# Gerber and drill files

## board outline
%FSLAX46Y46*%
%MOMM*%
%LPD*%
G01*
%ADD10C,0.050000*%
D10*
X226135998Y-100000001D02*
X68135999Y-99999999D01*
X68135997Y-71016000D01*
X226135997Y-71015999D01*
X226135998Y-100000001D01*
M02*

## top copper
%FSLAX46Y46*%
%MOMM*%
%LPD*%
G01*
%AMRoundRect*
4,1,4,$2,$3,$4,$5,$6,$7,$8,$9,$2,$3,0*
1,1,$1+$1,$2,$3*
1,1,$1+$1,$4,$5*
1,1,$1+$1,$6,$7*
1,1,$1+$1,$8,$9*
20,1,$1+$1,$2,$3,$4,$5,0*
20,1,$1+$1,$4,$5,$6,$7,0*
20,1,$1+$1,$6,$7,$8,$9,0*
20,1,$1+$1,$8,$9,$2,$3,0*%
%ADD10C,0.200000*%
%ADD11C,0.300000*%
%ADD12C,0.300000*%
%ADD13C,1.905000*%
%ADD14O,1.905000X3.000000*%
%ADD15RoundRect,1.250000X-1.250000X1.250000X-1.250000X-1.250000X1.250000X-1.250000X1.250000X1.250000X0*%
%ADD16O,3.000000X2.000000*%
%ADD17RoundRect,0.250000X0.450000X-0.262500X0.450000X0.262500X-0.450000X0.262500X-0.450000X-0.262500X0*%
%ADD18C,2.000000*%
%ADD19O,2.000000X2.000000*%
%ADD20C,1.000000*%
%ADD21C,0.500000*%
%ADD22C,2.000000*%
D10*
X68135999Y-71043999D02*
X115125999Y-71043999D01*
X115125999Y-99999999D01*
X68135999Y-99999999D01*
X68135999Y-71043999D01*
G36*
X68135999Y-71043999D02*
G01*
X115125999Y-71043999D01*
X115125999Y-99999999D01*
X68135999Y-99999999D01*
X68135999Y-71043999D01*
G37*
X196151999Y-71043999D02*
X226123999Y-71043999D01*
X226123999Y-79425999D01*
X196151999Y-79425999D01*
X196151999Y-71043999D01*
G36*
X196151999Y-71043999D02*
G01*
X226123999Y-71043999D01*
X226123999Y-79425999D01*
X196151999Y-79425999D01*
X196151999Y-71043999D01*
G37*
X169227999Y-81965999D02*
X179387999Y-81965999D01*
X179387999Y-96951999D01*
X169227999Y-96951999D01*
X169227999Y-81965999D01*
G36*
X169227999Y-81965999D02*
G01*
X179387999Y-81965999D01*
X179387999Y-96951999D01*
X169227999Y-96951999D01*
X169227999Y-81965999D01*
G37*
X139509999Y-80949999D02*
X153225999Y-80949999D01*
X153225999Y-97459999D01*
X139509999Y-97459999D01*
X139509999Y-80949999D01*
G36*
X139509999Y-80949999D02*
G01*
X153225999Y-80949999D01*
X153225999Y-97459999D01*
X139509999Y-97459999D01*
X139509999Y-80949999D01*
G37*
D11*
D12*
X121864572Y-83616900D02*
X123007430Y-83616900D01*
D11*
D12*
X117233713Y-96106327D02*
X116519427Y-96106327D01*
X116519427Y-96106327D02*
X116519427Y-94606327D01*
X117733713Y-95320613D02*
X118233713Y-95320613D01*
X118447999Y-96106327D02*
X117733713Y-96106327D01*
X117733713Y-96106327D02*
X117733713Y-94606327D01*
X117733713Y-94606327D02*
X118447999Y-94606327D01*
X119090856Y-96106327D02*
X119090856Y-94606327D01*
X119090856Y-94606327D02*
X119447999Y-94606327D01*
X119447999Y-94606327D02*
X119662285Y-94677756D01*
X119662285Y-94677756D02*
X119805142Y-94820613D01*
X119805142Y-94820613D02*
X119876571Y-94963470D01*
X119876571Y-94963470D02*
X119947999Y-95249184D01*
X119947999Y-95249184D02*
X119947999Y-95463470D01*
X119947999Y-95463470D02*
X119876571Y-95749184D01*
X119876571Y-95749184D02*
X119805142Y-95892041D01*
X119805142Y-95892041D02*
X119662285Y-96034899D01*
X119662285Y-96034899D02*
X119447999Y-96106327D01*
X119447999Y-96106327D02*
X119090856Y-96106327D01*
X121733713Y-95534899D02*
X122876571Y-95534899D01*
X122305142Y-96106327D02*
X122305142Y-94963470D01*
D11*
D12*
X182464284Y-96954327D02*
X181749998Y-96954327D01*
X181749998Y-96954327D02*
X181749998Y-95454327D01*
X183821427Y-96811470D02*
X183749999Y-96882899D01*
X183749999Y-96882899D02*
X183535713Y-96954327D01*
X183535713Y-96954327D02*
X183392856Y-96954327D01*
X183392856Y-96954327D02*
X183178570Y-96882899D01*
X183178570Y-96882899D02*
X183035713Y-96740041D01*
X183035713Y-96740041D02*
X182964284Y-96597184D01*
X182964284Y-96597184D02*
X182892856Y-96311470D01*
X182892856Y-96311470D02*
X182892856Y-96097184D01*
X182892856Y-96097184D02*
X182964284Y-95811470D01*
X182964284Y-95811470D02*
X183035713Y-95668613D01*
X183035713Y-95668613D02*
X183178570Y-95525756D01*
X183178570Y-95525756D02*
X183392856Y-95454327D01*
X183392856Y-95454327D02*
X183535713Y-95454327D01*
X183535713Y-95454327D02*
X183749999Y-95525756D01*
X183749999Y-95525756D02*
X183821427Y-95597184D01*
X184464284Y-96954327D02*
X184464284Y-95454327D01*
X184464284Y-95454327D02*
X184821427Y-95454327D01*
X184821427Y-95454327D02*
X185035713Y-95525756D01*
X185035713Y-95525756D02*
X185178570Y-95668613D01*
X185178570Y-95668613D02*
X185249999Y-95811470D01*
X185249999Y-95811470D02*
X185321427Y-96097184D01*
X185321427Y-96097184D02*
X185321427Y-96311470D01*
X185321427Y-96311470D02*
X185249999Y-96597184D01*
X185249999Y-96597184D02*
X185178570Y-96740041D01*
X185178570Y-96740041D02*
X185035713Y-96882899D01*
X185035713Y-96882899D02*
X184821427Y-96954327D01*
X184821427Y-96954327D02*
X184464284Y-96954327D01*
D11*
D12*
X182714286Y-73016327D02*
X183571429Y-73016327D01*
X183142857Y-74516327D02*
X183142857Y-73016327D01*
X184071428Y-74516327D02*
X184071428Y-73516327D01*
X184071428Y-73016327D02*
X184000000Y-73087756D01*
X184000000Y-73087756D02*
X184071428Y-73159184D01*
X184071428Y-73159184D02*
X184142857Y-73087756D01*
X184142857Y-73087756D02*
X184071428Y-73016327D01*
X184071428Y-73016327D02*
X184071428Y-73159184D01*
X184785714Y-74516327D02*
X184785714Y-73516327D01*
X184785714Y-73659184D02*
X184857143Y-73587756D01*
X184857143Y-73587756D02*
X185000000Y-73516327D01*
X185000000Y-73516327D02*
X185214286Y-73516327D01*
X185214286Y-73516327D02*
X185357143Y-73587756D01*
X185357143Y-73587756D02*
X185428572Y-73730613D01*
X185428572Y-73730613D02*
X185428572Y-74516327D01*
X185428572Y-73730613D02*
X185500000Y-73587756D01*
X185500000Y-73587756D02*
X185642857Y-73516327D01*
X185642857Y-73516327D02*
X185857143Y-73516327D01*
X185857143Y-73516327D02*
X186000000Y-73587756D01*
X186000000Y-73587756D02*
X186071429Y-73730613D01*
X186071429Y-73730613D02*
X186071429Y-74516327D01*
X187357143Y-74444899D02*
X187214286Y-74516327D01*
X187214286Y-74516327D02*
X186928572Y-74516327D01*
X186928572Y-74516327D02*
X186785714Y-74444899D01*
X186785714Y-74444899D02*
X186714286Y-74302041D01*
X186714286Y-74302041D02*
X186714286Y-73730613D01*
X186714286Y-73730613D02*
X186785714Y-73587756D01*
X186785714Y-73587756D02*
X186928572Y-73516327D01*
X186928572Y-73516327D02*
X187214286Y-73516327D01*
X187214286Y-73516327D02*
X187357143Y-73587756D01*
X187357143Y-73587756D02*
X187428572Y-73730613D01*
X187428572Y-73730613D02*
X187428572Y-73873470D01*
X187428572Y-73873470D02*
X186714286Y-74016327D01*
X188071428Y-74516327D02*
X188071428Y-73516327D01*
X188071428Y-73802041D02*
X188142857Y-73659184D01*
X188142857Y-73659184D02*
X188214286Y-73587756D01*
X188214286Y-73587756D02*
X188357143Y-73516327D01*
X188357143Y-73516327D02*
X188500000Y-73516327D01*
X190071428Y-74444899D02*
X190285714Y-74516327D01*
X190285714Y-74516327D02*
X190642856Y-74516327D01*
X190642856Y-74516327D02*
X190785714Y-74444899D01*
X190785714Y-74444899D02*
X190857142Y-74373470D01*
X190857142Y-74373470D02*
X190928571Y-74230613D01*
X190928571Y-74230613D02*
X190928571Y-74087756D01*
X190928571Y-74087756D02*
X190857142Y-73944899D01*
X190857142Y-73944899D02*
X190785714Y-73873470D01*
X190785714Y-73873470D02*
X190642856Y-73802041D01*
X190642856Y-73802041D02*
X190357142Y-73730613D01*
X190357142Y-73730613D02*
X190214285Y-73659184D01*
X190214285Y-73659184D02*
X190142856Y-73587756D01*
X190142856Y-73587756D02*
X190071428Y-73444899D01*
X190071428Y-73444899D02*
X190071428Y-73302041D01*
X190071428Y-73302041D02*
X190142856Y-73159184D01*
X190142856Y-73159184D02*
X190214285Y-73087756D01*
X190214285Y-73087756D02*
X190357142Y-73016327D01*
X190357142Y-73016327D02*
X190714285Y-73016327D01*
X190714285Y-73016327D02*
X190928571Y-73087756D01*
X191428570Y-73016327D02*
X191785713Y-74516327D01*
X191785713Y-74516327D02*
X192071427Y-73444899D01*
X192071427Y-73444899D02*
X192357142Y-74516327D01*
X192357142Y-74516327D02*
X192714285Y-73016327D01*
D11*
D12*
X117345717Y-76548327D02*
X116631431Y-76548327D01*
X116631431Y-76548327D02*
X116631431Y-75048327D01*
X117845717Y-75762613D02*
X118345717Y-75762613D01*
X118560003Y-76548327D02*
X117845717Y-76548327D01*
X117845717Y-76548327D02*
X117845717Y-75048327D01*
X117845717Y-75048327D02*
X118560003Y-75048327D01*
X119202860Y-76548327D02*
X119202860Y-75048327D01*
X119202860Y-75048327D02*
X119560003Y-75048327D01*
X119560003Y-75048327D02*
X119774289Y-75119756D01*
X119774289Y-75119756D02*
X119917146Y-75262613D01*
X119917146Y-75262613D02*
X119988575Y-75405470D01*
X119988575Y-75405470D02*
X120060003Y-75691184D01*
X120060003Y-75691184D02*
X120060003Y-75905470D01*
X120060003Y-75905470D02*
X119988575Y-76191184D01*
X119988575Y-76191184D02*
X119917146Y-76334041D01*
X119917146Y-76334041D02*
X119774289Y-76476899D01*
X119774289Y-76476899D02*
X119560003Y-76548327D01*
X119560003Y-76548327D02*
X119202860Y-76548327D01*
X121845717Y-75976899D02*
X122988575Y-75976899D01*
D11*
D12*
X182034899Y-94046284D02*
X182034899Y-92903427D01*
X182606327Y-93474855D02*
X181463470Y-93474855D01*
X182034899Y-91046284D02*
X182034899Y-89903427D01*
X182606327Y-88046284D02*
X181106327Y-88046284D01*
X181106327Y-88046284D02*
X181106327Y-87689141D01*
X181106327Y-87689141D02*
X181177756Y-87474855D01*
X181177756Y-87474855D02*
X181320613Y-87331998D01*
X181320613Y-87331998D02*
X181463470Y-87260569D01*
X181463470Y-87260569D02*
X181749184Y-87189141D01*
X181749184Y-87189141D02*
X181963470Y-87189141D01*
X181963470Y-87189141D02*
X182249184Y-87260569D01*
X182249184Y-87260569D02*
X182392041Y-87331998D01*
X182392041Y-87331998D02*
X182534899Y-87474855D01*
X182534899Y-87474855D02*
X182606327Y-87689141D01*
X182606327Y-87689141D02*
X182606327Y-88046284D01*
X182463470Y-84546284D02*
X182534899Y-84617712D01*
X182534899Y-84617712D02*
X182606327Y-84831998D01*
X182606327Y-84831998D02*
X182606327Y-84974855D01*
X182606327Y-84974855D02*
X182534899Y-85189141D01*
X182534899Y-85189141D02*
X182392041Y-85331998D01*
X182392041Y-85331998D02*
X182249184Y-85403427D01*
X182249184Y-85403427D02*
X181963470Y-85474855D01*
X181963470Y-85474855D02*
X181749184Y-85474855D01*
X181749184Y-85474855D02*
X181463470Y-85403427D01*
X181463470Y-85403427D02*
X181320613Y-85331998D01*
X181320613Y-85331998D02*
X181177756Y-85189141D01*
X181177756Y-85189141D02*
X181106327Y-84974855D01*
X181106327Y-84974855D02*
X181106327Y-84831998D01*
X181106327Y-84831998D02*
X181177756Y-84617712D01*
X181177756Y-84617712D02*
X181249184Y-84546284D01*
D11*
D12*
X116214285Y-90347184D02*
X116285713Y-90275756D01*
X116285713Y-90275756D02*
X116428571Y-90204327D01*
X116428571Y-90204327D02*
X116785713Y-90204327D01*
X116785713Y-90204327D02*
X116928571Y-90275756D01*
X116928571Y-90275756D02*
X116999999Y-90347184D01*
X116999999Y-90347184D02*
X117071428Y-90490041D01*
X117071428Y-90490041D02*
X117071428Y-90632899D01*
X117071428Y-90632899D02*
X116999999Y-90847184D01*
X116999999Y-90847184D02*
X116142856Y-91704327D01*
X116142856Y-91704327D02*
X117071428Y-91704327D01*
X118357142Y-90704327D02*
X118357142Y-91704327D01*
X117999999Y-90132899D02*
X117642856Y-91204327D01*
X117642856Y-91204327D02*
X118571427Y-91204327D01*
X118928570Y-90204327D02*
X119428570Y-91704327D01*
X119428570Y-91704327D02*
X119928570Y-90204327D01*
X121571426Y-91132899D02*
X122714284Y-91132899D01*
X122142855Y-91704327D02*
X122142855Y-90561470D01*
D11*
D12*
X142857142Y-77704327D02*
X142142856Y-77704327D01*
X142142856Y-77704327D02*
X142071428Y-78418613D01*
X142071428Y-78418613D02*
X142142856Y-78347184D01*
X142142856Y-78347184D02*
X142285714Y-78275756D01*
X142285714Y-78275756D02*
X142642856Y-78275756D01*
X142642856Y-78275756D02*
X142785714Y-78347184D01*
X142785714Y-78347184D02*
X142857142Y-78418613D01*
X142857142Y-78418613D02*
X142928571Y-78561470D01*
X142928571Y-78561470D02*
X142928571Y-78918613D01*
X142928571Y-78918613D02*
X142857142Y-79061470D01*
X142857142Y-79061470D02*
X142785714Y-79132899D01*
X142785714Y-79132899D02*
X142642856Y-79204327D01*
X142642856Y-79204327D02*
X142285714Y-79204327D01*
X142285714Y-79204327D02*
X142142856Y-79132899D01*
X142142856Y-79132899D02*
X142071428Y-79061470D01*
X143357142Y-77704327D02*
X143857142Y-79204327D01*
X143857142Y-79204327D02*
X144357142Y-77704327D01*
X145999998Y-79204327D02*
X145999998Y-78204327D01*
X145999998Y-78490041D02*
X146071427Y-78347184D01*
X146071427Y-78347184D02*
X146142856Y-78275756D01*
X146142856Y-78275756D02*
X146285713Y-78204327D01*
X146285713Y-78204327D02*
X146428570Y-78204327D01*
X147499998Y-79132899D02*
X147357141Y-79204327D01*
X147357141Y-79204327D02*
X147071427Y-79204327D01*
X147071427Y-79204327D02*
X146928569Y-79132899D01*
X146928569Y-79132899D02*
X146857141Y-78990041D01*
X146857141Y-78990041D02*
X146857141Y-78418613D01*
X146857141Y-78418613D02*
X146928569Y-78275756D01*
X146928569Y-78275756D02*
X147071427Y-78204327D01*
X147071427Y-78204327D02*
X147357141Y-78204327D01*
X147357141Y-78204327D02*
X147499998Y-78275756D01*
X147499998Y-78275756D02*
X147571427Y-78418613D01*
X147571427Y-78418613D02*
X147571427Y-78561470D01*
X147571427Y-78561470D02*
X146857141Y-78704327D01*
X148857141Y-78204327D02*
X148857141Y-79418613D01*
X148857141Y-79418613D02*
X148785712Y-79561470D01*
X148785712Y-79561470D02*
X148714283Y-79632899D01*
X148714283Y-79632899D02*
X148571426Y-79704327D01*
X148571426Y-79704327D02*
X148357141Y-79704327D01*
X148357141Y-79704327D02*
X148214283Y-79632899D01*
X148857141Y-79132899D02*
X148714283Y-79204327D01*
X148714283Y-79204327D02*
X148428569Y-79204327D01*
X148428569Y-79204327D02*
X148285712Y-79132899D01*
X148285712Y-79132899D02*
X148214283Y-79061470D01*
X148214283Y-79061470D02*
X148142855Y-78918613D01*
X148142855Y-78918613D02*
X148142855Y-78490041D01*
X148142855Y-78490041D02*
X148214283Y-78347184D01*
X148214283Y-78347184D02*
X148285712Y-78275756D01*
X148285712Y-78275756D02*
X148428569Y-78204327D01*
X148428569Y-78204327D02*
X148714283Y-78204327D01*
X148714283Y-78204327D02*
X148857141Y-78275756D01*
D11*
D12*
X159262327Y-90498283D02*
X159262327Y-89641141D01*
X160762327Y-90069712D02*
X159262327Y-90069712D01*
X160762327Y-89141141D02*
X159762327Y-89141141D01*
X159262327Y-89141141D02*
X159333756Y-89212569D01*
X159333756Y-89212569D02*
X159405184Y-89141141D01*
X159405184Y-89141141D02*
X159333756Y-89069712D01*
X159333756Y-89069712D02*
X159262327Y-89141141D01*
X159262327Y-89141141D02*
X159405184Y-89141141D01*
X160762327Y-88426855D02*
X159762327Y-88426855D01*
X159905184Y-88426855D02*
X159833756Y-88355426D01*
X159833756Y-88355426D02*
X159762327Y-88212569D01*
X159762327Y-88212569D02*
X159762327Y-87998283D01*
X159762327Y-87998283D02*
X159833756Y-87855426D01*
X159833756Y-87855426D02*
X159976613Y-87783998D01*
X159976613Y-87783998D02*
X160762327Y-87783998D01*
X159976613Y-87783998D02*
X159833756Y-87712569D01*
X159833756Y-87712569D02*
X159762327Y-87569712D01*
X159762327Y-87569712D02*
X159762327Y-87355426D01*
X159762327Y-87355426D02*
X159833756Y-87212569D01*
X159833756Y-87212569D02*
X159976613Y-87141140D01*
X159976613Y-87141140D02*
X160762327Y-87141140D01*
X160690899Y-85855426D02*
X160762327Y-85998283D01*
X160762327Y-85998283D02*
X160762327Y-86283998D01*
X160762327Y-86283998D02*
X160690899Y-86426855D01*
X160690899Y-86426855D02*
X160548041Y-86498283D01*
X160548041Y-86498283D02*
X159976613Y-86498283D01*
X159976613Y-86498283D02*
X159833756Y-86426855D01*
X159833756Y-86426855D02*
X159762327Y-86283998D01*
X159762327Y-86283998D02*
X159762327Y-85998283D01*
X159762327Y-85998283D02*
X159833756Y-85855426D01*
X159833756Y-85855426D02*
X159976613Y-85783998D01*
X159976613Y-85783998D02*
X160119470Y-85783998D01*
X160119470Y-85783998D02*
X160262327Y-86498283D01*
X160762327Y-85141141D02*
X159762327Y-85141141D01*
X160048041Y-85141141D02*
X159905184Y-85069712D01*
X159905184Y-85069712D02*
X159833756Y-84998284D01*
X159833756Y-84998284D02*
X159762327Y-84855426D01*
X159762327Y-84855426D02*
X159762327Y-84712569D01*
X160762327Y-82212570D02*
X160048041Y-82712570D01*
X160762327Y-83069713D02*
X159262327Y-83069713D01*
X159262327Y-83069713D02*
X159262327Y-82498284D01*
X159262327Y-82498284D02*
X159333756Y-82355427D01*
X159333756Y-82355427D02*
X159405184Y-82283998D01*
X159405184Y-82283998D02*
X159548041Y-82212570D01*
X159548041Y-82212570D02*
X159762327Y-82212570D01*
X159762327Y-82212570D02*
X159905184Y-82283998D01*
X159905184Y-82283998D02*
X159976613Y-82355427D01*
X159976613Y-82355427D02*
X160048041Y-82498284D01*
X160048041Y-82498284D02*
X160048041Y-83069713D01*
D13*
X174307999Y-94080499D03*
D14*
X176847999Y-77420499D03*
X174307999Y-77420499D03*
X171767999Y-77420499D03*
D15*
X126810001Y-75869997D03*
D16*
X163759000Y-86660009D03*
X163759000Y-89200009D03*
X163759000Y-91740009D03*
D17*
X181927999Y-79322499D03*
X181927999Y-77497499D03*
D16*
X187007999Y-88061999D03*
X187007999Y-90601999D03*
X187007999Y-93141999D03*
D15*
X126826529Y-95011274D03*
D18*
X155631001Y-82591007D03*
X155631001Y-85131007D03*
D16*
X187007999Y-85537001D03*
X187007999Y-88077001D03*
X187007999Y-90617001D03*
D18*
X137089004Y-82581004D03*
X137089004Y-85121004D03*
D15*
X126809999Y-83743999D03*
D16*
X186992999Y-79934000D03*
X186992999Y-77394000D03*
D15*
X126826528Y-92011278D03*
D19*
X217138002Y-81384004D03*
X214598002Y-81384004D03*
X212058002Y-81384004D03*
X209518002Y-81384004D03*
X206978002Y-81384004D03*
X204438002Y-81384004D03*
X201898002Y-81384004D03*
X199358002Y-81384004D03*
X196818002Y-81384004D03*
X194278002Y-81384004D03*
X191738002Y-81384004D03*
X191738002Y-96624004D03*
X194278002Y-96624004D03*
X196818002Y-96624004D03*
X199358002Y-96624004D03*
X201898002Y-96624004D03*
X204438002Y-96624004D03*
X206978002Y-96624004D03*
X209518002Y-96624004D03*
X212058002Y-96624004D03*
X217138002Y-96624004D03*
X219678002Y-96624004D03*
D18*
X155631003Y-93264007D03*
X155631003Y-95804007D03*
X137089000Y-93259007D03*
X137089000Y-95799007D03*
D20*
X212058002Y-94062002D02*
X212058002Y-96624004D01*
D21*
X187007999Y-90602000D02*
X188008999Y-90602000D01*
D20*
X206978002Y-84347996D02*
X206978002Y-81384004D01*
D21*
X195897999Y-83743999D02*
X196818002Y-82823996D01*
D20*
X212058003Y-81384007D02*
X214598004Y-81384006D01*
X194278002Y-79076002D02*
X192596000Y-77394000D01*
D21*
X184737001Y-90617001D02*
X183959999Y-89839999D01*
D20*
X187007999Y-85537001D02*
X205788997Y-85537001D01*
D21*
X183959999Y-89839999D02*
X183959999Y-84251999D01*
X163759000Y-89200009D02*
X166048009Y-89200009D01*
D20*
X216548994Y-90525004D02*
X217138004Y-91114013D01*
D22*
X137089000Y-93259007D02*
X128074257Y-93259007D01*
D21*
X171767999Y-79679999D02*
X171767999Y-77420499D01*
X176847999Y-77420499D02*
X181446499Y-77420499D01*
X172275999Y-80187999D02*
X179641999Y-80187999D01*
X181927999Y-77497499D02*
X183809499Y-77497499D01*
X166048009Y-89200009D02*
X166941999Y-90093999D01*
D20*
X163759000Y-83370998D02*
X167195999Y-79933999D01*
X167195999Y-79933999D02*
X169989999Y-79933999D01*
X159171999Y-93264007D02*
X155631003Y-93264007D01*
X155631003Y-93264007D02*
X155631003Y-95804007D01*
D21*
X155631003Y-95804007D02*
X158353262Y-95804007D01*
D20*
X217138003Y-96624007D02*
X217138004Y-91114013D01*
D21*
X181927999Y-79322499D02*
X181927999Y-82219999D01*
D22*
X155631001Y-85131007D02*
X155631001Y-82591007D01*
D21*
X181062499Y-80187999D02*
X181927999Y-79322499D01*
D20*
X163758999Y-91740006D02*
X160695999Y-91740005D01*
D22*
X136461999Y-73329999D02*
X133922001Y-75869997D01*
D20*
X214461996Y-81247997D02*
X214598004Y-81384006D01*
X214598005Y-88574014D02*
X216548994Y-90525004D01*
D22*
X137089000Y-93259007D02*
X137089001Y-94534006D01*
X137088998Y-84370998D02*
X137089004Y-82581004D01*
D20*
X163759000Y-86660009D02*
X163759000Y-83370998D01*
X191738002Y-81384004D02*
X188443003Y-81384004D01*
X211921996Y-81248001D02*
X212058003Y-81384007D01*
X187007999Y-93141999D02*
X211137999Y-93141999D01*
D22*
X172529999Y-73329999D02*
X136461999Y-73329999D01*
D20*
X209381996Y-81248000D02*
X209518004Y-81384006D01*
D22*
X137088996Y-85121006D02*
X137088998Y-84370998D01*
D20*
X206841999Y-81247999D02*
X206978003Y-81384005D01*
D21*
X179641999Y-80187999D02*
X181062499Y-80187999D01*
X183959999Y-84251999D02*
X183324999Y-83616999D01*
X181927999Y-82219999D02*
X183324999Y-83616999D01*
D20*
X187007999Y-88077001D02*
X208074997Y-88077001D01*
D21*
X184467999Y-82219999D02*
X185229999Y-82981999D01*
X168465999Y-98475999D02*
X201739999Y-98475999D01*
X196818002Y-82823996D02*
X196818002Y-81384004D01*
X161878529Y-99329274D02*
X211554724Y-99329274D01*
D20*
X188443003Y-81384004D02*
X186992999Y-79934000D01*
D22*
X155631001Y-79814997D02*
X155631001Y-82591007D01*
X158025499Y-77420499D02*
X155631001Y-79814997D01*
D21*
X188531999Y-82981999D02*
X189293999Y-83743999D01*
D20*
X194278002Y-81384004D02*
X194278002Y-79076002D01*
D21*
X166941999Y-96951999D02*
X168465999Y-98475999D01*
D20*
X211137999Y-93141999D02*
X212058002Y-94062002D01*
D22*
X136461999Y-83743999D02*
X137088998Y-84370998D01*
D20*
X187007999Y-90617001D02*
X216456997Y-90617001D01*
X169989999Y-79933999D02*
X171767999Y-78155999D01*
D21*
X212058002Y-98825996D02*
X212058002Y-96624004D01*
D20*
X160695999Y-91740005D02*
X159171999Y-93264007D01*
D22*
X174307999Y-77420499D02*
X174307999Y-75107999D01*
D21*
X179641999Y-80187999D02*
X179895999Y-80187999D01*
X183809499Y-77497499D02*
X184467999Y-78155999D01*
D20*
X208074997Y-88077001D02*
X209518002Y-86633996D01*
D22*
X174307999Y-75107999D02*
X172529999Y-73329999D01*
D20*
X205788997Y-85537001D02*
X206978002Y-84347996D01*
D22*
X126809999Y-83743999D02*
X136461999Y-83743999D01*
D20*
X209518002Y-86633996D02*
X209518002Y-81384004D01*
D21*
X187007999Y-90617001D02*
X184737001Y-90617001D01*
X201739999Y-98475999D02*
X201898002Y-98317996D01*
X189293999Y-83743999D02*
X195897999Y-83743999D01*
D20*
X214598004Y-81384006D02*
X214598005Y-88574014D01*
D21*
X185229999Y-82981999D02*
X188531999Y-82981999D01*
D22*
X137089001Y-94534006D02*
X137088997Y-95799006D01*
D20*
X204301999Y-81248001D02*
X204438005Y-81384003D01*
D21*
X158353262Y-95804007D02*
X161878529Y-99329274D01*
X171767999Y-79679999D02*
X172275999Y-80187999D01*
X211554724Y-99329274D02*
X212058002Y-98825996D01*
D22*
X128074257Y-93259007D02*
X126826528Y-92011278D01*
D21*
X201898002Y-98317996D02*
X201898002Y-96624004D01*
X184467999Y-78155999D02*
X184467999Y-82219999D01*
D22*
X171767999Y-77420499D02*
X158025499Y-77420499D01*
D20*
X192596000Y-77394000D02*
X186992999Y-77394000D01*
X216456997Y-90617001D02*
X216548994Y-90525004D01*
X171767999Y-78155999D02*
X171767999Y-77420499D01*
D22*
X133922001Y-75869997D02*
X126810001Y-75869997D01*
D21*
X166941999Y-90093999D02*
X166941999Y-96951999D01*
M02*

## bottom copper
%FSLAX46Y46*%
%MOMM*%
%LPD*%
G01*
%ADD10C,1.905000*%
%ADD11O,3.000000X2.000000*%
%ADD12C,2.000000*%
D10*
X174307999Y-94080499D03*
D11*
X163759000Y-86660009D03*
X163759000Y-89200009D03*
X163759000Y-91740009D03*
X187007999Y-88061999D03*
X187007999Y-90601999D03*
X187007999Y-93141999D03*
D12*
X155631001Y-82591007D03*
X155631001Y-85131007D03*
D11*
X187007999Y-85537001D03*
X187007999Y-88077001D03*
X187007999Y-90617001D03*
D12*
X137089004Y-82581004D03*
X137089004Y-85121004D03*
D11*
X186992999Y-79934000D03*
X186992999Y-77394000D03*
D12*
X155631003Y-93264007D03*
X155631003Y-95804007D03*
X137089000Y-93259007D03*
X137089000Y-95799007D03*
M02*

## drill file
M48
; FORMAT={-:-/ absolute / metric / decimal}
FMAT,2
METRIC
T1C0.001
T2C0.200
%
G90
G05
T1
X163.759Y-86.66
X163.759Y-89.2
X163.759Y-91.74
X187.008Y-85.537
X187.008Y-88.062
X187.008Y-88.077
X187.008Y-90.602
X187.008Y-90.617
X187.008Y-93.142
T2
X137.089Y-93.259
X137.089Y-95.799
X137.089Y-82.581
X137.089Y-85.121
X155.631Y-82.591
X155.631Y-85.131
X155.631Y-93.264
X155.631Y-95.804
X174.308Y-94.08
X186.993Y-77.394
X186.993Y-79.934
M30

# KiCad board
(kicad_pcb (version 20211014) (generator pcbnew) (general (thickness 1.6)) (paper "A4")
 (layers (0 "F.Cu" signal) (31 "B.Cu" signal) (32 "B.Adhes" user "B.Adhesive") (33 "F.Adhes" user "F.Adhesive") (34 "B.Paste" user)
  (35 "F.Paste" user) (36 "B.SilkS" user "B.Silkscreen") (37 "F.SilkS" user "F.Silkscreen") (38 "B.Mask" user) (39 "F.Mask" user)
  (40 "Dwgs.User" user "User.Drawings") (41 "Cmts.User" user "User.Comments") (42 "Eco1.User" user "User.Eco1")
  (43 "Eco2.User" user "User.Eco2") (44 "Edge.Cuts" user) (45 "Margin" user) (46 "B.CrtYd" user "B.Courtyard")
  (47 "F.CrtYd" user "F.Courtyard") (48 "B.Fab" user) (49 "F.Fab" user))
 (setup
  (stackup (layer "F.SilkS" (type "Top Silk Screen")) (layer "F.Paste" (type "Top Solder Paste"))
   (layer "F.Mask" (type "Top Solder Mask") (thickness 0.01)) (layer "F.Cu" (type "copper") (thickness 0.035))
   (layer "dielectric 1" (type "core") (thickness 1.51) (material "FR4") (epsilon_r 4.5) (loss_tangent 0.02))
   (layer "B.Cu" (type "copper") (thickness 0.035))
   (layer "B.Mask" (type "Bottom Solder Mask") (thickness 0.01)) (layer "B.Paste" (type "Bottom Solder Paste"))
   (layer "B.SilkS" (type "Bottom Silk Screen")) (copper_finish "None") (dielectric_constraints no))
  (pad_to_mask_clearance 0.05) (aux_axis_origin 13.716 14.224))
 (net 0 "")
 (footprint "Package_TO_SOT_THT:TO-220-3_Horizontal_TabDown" (layer "F.Cu") (at 176.847999 77.420499 180)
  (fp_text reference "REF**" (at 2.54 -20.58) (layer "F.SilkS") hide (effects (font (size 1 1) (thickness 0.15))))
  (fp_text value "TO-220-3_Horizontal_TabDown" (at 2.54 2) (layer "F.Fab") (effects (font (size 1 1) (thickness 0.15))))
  (pad "" thru_hole circle (at 2.54 -16.66 180) (size 1.905 1.905) (drill 0.2) (layers *.Cu *.Mask))
  (pad "1" smd oval (at 0 0 180) (size 1.905 3) (layers "F.Cu" "F.Paste" "F.Mask"))
  (pad "2" smd oval (at 2.54 0 180) (size 1.905 3) (layers "F.Cu" "F.Paste" "F.Mask"))
  (pad "3" smd oval (at 5.08 0 180) (size 1.905 3) (layers "F.Cu" "F.Paste" "F.Mask")))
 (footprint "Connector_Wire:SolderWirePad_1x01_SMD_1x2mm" (layer "F.Cu") (at 126.810001 75.869997 -90)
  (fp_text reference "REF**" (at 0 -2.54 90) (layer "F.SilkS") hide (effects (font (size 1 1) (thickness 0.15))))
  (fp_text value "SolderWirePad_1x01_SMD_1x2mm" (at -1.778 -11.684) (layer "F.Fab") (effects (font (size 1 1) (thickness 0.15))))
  (pad "1" smd roundrect locked (at 0 0 270) (size 5 5) (layers "F.Cu" "F.Paste" "F.Mask") (roundrect_rratio 0.25)))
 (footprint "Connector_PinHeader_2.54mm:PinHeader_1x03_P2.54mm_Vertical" (layer "F.Cu") (at 163.759 86.660009)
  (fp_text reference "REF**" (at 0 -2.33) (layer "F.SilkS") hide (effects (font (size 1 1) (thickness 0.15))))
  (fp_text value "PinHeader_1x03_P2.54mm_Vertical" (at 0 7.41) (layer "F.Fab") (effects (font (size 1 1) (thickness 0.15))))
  (pad "1" thru_hole oval locked (at 0 0) (size 3 2) (drill 0.001) (layers *.Cu *.Mask))
  (pad "2" thru_hole oval locked (at 0 2.54) (size 3 2) (drill 0.001) (layers *.Cu *.Mask))
  (pad "3" thru_hole oval locked (at 0 5.08) (size 3 2) (drill 0.001) (layers *.Cu *.Mask)))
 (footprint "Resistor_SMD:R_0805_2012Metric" (layer "F.Cu") (at 181.927999 78.409999 90)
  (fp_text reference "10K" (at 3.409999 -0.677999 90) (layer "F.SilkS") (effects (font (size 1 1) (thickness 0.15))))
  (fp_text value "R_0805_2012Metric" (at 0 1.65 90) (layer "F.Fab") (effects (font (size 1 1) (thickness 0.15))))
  (pad "1" smd roundrect (at -0.9125 0 90) (size 1.025 1.4) (layers "F.Cu" "F.Paste" "F.Mask") (roundrect_rratio 0.243902))
  (pad "2" smd roundrect (at 0.9125 0 90) (size 1.025 1.4) (layers "F.Cu" "F.Paste" "F.Mask") (roundrect_rratio 0.243902)))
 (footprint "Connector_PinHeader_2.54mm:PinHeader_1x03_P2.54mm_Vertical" (layer "F.Cu") (at 187.007999 88.061999)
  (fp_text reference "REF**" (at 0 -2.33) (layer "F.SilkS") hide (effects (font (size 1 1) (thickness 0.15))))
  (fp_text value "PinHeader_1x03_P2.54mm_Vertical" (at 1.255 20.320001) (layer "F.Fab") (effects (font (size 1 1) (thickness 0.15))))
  (pad "1" thru_hole oval locked (at 0 0) (size 3 2) (drill 0.001) (layers *.Cu *.Mask))
  (pad "2" thru_hole oval locked (at 0 2.54) (size 3 2) (drill 0.001) (layers *.Cu *.Mask))
  (pad "3" thru_hole oval locked (at 0 5.08) (size 3 2) (drill 0.001) (layers *.Cu *.Mask)))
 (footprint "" (layer "F.Cu") (at 126.826529 95.011274)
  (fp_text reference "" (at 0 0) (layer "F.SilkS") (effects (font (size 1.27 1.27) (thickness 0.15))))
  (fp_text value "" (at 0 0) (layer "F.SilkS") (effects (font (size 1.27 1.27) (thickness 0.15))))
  (pad "1" smd roundrect locked (at 0 0 270) (size 5 5) (layers "F.Cu" "F.Paste" "F.Mask") (roundrect_rratio 0.25)))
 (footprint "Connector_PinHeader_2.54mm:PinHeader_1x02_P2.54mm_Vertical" (layer "F.Cu") (at 155.631001 82.591007)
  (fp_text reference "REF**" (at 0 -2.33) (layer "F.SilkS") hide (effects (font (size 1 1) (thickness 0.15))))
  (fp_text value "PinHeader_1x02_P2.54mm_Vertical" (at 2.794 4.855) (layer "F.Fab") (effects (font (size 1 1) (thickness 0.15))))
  (pad "1" thru_hole circle (at 0 0) (size 2 2) (drill 0.2) (layers *.Cu *.Mask))
  (pad "2" thru_hole circle (at 0 2.54) (size 2 2) (drill 0.2) (layers *.Cu *.Mask)))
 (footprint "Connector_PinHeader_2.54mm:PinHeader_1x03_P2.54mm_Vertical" (layer "F.Cu") (at 187.007999 85.537001)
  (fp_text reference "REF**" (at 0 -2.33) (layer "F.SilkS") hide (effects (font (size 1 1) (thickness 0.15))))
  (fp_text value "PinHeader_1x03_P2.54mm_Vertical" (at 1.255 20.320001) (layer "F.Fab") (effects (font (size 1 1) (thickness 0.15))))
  (pad "1" thru_hole oval locked (at 0 0) (size 3 2) (drill 0.001) (layers *.Cu *.Mask))
  (pad "2" thru_hole oval locked (at 0 2.54) (size 3 2) (drill 0.001) (layers *.Cu *.Mask))
  (pad "3" thru_hole oval locked (at 0 5.08) (size 3 2) (drill 0.001) (layers *.Cu *.Mask)))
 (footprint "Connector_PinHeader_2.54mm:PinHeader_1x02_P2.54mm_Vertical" (layer "F.Cu") (at 137.089004 82.581004)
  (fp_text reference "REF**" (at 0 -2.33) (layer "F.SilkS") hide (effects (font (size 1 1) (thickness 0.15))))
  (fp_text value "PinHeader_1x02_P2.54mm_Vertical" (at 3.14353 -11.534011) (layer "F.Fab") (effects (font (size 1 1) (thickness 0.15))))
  (pad "1" thru_hole circle (at 0 0) (size 2 2) (drill 0.2) (layers *.Cu *.Mask))
  (pad "2" thru_hole circle (at 0 2.54) (size 2 2) (drill 0.2) (layers *.Cu *.Mask)))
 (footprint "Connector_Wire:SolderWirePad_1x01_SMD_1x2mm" (layer "F.Cu") (at 126.809999 83.743999 -90)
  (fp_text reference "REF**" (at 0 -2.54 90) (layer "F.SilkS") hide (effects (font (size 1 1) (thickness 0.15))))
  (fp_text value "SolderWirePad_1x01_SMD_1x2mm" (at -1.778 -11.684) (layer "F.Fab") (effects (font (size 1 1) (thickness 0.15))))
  (pad "1" smd roundrect locked (at 0 0 270) (size 5 5) (layers "F.Cu" "F.Paste" "F.Mask") (roundrect_rratio 0.25)))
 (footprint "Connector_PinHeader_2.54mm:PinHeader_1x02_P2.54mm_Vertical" (layer "F.Cu") (at 186.992999 79.934 180)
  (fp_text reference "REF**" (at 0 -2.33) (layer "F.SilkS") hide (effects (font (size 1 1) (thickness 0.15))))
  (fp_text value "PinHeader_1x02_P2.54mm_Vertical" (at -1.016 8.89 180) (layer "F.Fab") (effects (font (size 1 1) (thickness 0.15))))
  (pad "1" thru_hole oval (at 0 0 180) (size 3 2) (drill 0.2) (layers *.Cu *.Mask))
  (pad "2" thru_hole oval (at 0 2.54 180) (size 3 2) (drill 0.2) (layers *.Cu *.Mask)))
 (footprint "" (layer "F.Cu") (at 126.826528 92.011278)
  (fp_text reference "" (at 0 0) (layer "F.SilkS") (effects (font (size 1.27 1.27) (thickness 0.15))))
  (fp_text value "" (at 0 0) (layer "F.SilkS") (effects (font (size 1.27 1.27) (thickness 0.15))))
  (pad "1" smd roundrect locked (at 0 0 270) (size 5 5) (layers "F.Cu" "F.Paste" "F.Mask") (roundrect_rratio 0.25)))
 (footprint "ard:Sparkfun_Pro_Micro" (layer "F.Cu") (at 191.738002 96.624004 90)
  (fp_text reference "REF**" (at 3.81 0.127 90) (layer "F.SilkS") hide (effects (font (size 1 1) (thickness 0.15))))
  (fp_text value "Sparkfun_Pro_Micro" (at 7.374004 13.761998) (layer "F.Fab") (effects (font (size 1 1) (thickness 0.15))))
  (pad "" smd oval locked (at 0 22.86 90) (size 2 2) (layers "F.Paste" "F.Mask"))
  (pad "" smd oval locked (at 15.24 27.94 90) (size 2 2) (layers "F.Paste" "F.Mask"))
  (pad "2" smd oval locked (at 15.24 25.4 90) (size 2 2) (layers "F.Cu" "F.Paste" "F.Mask"))
  (pad "3" smd oval locked (at 15.24 22.86 90) (size 2 2) (layers "F.Cu" "F.Paste" "F.Mask"))
  (pad "4" smd oval locked (at 15.24 20.32 90) (size 2 2) (layers "F.Cu" "F.Paste" "F.Mask"))
  (pad "5" smd oval locked (at 15.24 17.78 90) (size 2 2) (layers "F.Cu" "F.Paste" "F.Mask"))
  (pad "6" smd oval locked (at 15.24 15.24 90) (size 2 2) (layers "F.Cu" "F.Paste" "F.Mask"))
  (pad "7" smd oval locked (at 15.24 12.7 90) (size 2 2) (layers "F.Cu" "F.Paste" "F.Mask"))
  (pad "8" smd oval locked (at 15.24 10.16 90) (size 2 2) (layers "F.Cu" "F.Paste" "F.Mask"))
  (pad "9" smd oval locked (at 15.24 7.62 90) (size 2 2) (layers "F.Cu" "F.Paste" "F.Mask"))
  (pad "10" smd oval locked (at 15.24 5.08 90) (size 2 2) (layers "F.Cu" "F.Paste" "F.Mask"))
  (pad "11" smd oval locked (at 15.24 2.54 90) (size 2 2) (layers "F.Cu" "F.Paste" "F.Mask"))
  (pad "12" smd oval locked (at 15.24 0 90) (size 2 2) (layers "F.Cu" "F.Paste" "F.Mask"))
  (pad "13" smd oval locked (at 0 0 90) (size 2 2) (layers "F.Cu" "F.Paste" "F.Mask"))
  (pad "14" smd oval locked (at 0 2.54 90) (size 2 2) (layers "F.Cu" "F.Paste" "F.Mask"))
  (pad "15" smd oval locked (at 0 5.08 90) (size 2 2) (layers "F.Cu" "F.Paste" "F.Mask"))
  (pad "16" smd oval locked (at 0 7.62 90) (size 2 2) (layers "F.Cu" "F.Paste" "F.Mask"))
  (pad "17" smd oval locked (at 0 10.16 90) (size 2 2) (layers "F.Cu" "F.Paste" "F.Mask"))
  (pad "18" smd oval locked (at 0 12.7 90) (size 2 2) (layers "F.Cu" "F.Paste" "F.Mask"))
  (pad "19" smd oval locked (at 0 15.24 90) (size 2 2) (layers "F.Cu" "F.Paste" "F.Mask"))
  (pad "20" smd oval locked (at 0 17.78 90) (size 2 2) (layers "F.Cu" "F.Paste" "F.Mask"))
  (pad "21" smd oval locked (at 0 20.32 90) (size 2 2) (layers "F.Cu" "F.Paste" "F.Mask"))
  (pad "23" smd oval locked (at 0 25.4 90) (size 2 2) (layers "F.Cu" "F.Paste" "F.Mask"))
  (pad "24" smd oval locked (at 0 27.94 90) (size 2 2) (layers "F.Cu" "F.Paste" "F.Mask")))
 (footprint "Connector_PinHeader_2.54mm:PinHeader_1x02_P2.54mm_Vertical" (layer "F.Cu") (at 155.631003 93.264007)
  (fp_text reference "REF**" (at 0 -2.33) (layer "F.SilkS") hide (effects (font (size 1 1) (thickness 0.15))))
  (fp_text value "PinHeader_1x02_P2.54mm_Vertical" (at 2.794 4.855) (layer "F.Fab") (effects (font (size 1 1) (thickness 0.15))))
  (pad "1" thru_hole circle (at 0 0) (size 2 2) (drill 0.2) (layers *.Cu *.Mask))
  (pad "2" thru_hole circle (at 0 2.54) (size 2 2) (drill 0.2) (layers *.Cu *.Mask)))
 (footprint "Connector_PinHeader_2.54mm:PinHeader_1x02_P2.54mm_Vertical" (layer "F.Cu") (at 137.089 93.259007)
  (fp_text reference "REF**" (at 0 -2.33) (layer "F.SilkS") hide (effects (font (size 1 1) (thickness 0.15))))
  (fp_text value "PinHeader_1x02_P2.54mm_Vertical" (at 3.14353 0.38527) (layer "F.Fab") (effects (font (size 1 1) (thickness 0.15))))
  (pad "1" thru_hole circle (at 0 0) (size 2 2) (drill 0.2) (layers *.Cu *.Mask))
  (pad "2" thru_hole circle (at 0 2.54) (size 2 2) (drill 0.2) (layers *.Cu *.Mask)))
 (gr_rect (start 68.135999 71.043999) (end 115.125999 99.999999) (layer "F.Cu") (width 0.2) (fill solid))
 (gr_rect (start 196.151999 71.043999) (end 226.123999 79.425999) (layer "F.Cu") (width 0.2) (fill solid))
 (gr_rect (start 169.227999 96.951999) (end 179.387999 81.965999) (layer "F.Cu") (width 0.2) (fill solid))
 (gr_rect (start 139.509999 80.949999) (end 153.225999 97.459999) (layer "F.Cu") (width 0.2) (fill solid))
 (gr_poly
  (pts (xy 226.135998 100.000001) (xy 68.135999 99.999999) (xy 68.135997 71.016) (xy 226.135997 71.015999)) (layer "Edge.Cuts") (width 0.05)
  (fill none))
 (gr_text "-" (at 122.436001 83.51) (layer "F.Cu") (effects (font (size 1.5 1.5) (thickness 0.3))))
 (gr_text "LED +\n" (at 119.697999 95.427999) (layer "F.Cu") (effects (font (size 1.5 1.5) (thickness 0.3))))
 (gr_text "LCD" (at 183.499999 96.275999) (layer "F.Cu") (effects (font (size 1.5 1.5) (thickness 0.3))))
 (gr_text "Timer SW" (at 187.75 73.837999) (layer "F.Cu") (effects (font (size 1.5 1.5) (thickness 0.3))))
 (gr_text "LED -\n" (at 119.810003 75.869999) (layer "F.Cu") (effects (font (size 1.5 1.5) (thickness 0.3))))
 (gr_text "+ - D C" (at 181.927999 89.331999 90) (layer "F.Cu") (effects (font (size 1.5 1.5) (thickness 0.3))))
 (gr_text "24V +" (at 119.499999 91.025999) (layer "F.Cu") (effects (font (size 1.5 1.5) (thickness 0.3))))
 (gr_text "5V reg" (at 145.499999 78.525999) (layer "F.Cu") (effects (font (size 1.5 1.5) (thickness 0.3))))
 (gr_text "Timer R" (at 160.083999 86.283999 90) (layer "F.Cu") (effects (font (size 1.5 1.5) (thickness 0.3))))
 (segment (start 212.058002 94.062002) (end 212.058002 96.624004) (width 1) (layer "F.Cu") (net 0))
 (segment (start 187.007999 90.602) (end 188.008999 90.602) (width 0.5) (layer "F.Cu") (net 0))
 (segment (start 206.978002 84.347996) (end 206.978002 81.384004) (width 1) (layer "F.Cu") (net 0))
 (segment (start 195.897999 83.743999) (end 196.818002 82.823996) (width 0.5) (layer "F.Cu") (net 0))
 (segment (start 212.058003 81.384007) (end 214.598004 81.384006) (width 1) (layer "F.Cu") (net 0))
 (segment (start 194.278002 79.076002) (end 192.596 77.394) (width 1) (layer "F.Cu") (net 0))
 (segment (start 184.737001 90.617001) (end 183.959999 89.839999) (width 0.5) (layer "F.Cu") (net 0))
 (segment (start 187.007999 85.537001) (end 205.788997 85.537001) (width 1) (layer "F.Cu") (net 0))
 (segment (start 183.959999 89.839999) (end 183.959999 84.251999) (width 0.5) (layer "F.Cu") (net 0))
 (segment (start 163.759 89.200009) (end 166.048009 89.200009) (width 0.5) (layer "F.Cu") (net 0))
 (segment (start 216.548994 90.525004) (end 217.138004 91.114013) (width 1) (layer "F.Cu") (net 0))
 (segment (start 137.089 93.259007) (end 128.074257 93.259007) (width 2) (layer "F.Cu") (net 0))
 (segment (start 171.767999 79.679999) (end 171.767999 77.420499) (width 0.5) (layer "F.Cu") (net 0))
 (segment (start 176.847999 77.420499) (end 181.446499 77.420499) (width 0.5) (layer "F.Cu") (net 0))
 (segment (start 172.275999 80.187999) (end 179.641999 80.187999) (width 0.5) (layer "F.Cu") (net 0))
 (segment (start 181.927999 77.497499) (end 183.809499 77.497499) (width 0.5) (layer "F.Cu") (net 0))
 (segment (start 166.048009 89.200009) (end 166.941999 90.093999) (width 0.5) (layer "F.Cu") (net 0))
 (segment (start 163.759 83.370998) (end 167.195999 79.933999) (width 1) (layer "F.Cu") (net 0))
 (segment (start 167.195999 79.933999) (end 169.989999 79.933999) (width 1) (layer "F.Cu") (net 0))
 (segment (start 159.171999 93.264007) (end 155.631003 93.264007) (width 1) (layer "F.Cu") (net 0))
 (segment (start 155.631003 93.264007) (end 155.631003 95.804007) (width 1) (layer "F.Cu") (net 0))
 (segment (start 155.631003 95.804007) (end 158.353262 95.804007) (width 0.5) (layer "F.Cu") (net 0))
 (segment (start 217.138003 96.624007) (end 217.138004 91.114013) (width 1) (layer "F.Cu") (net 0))
 (segment (start 181.927999 79.322499) (end 181.927999 82.219999) (width 0.5) (layer "F.Cu") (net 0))
 (segment (start 155.631001 85.131007) (end 155.631001 82.591007) (width 2) (layer "F.Cu") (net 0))
 (segment (start 181.062499 80.187999) (end 181.927999 79.322499) (width 0.5) (layer "F.Cu") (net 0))
 (segment (start 163.758999 91.740006) (end 160.695999 91.740005) (width 1) (layer "F.Cu") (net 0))
 (segment (start 136.461999 73.329999) (end 133.922001 75.869997) (width 2) (layer "F.Cu") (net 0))
 (segment (start 214.461996 81.247997) (end 214.598004 81.384006) (width 1) (layer "F.Cu") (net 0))
 (segment (start 214.598005 88.574014) (end 216.548994 90.525004) (width 1) (layer "F.Cu") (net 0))
 (segment (start 137.089 93.259007) (end 137.089001 94.534006) (width 2) (layer "F.Cu") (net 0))
 (segment (start 137.088998 84.370998) (end 137.089004 82.581004) (width 2) (layer "F.Cu") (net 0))
 (segment (start 163.759 86.660009) (end 163.759 83.370998) (width 1) (layer "F.Cu") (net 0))
 (segment (start 191.738002 81.384004) (end 188.443003 81.384004) (width 1) (layer "F.Cu") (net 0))
 (segment (start 211.921996 81.248001) (end 212.058003 81.384007) (width 1) (layer "F.Cu") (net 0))
 (segment (start 187.007999 93.141999) (end 211.137999 93.141999) (width 1) (layer "F.Cu") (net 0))
 (segment (start 172.529999 73.329999) (end 136.461999 73.329999) (width 2) (layer "F.Cu") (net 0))
 (segment (start 209.381996 81.248) (end 209.518004 81.384006) (width 1) (layer "F.Cu") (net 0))
 (segment (start 137.088996 85.121006) (end 137.088998 84.370998) (width 2) (layer "F.Cu") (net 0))
 (segment (start 206.841999 81.247999) (end 206.978003 81.384005) (width 1) (layer "F.Cu") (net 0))
 (segment (start 179.641999 80.187999) (end 181.062499 80.187999) (width 0.5) (layer "F.Cu") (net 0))
 (segment (start 183.959999 84.251999) (end 183.324999 83.616999) (width 0.5) (layer "F.Cu") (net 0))
 (segment (start 181.927999 82.219999) (end 183.324999 83.616999) (width 0.5) (layer "F.Cu") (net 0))
 (segment (start 187.007999 88.077001) (end 208.074997 88.077001) (width 1) (layer "F.Cu") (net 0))
 (segment (start 184.467999 82.219999) (end 185.229999 82.981999) (width 0.5) (layer "F.Cu") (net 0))
 (segment (start 168.465999 98.475999) (end 201.739999 98.475999) (width 0.5) (layer "F.Cu") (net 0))
 (segment (start 196.818002 82.823996) (end 196.818002 81.384004) (width 0.5) (layer "F.Cu") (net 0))
 (segment (start 161.878529 99.329274) (end 211.554724 99.329274) (width 0.5) (layer "F.Cu") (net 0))
 (segment (start 188.443003 81.384004) (end 186.992999 79.934) (width 1) (layer "F.Cu") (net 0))
 (segment (start 155.631001 79.814997) (end 155.631001 82.591007) (width 2) (layer "F.Cu") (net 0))
 (segment (start 158.025499 77.420499) (end 155.631001 79.814997) (width 2) (layer "F.Cu") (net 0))
 (segment (start 188.531999 82.981999) (end 189.293999 83.743999) (width 0.5) (layer "F.Cu") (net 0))
 (segment (start 194.278002 81.384004) (end 194.278002 79.076002) (width 1) (layer "F.Cu") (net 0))
 (segment (start 166.941999 96.951999) (end 168.465999 98.475999) (width 0.5) (layer "F.Cu") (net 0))
 (segment (start 211.137999 93.141999) (end 212.058002 94.062002) (width 1) (layer "F.Cu") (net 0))
 (segment (start 136.461999 83.743999) (end 137.088998 84.370998) (width 2) (layer "F.Cu") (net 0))
 (segment (start 187.007999 90.617001) (end 216.456997 90.617001) (width 1) (layer "F.Cu") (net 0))
 (segment (start 169.989999 79.933999) (end 171.767999 78.155999) (width 1) (layer "F.Cu") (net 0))
 (segment (start 212.058002 98.825996) (end 212.058002 96.624004) (width 0.5) (layer "F.Cu") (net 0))
 (segment (start 160.695999 91.740005) (end 159.171999 93.264007) (width 1) (layer "F.Cu") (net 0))
 (segment (start 174.307999 77.420499) (end 174.307999 75.107999) (width 2) (layer "F.Cu") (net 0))
 (segment (start 179.641999 80.187999) (end 179.895999 80.187999) (width 0.5) (layer "F.Cu") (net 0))
 (segment (start 183.809499 77.497499) (end 184.467999 78.155999) (width 0.5) (layer "F.Cu") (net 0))
 (segment (start 208.074997 88.077001) (end 209.518002 86.633996) (width 1) (layer "F.Cu") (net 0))
 (segment (start 174.307999 75.107999) (end 172.529999 73.329999) (width 2) (layer "F.Cu") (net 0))
 (segment (start 205.788997 85.537001) (end 206.978002 84.347996) (width 1) (layer "F.Cu") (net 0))
 (segment (start 126.809999 83.743999) (end 136.461999 83.743999) (width 2) (layer "F.Cu") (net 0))
 (segment (start 209.518002 86.633996) (end 209.518002 81.384004) (width 1) (layer "F.Cu") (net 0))
 (segment (start 187.007999 90.617001) (end 184.737001 90.617001) (width 0.5) (layer "F.Cu") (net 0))
 (segment (start 201.739999 98.475999) (end 201.898002 98.317996) (width 0.5) (layer "F.Cu") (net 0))
 (segment (start 189.293999 83.743999) (end 195.897999 83.743999) (width 0.5) (layer "F.Cu") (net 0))
 (segment (start 214.598004 81.384006) (end 214.598005 88.574014) (width 1) (layer "F.Cu") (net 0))
 (segment (start 185.229999 82.981999) (end 188.531999 82.981999) (width 0.5) (layer "F.Cu") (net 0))
 (segment (start 137.089001 94.534006) (end 137.088997 95.799006) (width 2) (layer "F.Cu") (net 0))
 (segment (start 204.301999 81.248001) (end 204.438005 81.384003) (width 1) (layer "F.Cu") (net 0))
 (segment (start 158.353262 95.804007) (end 161.878529 99.329274) (width 0.5) (layer "F.Cu") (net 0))
 (segment (start 171.767999 79.679999) (end 172.275999 80.187999) (width 0.5) (layer "F.Cu") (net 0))
 (segment (start 211.554724 99.329274) (end 212.058002 98.825996) (width 0.5) (layer "F.Cu") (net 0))
 (segment (start 128.074257 93.259007) (end 126.826528 92.011278) (width 2) (layer "F.Cu") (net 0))
 (segment (start 201.898002 98.317996) (end 201.898002 96.624004) (width 0.5) (layer "F.Cu") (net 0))
 (segment (start 184.467999 78.155999) (end 184.467999 82.219999) (width 0.5) (layer "F.Cu") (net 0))
 (segment (start 171.767999 77.420499) (end 158.025499 77.420499) (width 2) (layer "F.Cu") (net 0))
 (segment (start 192.596 77.394) (end 186.992999 77.394) (width 1) (layer "F.Cu") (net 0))
 (segment (start 216.456997 90.617001) (end 216.548994 90.525004) (width 1) (layer "F.Cu") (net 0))
 (segment (start 171.767999 78.155999) (end 171.767999 77.420499) (width 1) (layer "F.Cu") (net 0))
 (segment (start 133.922001 75.869997) (end 126.810001 75.869997) (width 2) (layer "F.Cu") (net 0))
 (segment (start 166.941999 90.093999) (end 166.941999 96.951999) (width 0.5) (layer "F.Cu") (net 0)))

